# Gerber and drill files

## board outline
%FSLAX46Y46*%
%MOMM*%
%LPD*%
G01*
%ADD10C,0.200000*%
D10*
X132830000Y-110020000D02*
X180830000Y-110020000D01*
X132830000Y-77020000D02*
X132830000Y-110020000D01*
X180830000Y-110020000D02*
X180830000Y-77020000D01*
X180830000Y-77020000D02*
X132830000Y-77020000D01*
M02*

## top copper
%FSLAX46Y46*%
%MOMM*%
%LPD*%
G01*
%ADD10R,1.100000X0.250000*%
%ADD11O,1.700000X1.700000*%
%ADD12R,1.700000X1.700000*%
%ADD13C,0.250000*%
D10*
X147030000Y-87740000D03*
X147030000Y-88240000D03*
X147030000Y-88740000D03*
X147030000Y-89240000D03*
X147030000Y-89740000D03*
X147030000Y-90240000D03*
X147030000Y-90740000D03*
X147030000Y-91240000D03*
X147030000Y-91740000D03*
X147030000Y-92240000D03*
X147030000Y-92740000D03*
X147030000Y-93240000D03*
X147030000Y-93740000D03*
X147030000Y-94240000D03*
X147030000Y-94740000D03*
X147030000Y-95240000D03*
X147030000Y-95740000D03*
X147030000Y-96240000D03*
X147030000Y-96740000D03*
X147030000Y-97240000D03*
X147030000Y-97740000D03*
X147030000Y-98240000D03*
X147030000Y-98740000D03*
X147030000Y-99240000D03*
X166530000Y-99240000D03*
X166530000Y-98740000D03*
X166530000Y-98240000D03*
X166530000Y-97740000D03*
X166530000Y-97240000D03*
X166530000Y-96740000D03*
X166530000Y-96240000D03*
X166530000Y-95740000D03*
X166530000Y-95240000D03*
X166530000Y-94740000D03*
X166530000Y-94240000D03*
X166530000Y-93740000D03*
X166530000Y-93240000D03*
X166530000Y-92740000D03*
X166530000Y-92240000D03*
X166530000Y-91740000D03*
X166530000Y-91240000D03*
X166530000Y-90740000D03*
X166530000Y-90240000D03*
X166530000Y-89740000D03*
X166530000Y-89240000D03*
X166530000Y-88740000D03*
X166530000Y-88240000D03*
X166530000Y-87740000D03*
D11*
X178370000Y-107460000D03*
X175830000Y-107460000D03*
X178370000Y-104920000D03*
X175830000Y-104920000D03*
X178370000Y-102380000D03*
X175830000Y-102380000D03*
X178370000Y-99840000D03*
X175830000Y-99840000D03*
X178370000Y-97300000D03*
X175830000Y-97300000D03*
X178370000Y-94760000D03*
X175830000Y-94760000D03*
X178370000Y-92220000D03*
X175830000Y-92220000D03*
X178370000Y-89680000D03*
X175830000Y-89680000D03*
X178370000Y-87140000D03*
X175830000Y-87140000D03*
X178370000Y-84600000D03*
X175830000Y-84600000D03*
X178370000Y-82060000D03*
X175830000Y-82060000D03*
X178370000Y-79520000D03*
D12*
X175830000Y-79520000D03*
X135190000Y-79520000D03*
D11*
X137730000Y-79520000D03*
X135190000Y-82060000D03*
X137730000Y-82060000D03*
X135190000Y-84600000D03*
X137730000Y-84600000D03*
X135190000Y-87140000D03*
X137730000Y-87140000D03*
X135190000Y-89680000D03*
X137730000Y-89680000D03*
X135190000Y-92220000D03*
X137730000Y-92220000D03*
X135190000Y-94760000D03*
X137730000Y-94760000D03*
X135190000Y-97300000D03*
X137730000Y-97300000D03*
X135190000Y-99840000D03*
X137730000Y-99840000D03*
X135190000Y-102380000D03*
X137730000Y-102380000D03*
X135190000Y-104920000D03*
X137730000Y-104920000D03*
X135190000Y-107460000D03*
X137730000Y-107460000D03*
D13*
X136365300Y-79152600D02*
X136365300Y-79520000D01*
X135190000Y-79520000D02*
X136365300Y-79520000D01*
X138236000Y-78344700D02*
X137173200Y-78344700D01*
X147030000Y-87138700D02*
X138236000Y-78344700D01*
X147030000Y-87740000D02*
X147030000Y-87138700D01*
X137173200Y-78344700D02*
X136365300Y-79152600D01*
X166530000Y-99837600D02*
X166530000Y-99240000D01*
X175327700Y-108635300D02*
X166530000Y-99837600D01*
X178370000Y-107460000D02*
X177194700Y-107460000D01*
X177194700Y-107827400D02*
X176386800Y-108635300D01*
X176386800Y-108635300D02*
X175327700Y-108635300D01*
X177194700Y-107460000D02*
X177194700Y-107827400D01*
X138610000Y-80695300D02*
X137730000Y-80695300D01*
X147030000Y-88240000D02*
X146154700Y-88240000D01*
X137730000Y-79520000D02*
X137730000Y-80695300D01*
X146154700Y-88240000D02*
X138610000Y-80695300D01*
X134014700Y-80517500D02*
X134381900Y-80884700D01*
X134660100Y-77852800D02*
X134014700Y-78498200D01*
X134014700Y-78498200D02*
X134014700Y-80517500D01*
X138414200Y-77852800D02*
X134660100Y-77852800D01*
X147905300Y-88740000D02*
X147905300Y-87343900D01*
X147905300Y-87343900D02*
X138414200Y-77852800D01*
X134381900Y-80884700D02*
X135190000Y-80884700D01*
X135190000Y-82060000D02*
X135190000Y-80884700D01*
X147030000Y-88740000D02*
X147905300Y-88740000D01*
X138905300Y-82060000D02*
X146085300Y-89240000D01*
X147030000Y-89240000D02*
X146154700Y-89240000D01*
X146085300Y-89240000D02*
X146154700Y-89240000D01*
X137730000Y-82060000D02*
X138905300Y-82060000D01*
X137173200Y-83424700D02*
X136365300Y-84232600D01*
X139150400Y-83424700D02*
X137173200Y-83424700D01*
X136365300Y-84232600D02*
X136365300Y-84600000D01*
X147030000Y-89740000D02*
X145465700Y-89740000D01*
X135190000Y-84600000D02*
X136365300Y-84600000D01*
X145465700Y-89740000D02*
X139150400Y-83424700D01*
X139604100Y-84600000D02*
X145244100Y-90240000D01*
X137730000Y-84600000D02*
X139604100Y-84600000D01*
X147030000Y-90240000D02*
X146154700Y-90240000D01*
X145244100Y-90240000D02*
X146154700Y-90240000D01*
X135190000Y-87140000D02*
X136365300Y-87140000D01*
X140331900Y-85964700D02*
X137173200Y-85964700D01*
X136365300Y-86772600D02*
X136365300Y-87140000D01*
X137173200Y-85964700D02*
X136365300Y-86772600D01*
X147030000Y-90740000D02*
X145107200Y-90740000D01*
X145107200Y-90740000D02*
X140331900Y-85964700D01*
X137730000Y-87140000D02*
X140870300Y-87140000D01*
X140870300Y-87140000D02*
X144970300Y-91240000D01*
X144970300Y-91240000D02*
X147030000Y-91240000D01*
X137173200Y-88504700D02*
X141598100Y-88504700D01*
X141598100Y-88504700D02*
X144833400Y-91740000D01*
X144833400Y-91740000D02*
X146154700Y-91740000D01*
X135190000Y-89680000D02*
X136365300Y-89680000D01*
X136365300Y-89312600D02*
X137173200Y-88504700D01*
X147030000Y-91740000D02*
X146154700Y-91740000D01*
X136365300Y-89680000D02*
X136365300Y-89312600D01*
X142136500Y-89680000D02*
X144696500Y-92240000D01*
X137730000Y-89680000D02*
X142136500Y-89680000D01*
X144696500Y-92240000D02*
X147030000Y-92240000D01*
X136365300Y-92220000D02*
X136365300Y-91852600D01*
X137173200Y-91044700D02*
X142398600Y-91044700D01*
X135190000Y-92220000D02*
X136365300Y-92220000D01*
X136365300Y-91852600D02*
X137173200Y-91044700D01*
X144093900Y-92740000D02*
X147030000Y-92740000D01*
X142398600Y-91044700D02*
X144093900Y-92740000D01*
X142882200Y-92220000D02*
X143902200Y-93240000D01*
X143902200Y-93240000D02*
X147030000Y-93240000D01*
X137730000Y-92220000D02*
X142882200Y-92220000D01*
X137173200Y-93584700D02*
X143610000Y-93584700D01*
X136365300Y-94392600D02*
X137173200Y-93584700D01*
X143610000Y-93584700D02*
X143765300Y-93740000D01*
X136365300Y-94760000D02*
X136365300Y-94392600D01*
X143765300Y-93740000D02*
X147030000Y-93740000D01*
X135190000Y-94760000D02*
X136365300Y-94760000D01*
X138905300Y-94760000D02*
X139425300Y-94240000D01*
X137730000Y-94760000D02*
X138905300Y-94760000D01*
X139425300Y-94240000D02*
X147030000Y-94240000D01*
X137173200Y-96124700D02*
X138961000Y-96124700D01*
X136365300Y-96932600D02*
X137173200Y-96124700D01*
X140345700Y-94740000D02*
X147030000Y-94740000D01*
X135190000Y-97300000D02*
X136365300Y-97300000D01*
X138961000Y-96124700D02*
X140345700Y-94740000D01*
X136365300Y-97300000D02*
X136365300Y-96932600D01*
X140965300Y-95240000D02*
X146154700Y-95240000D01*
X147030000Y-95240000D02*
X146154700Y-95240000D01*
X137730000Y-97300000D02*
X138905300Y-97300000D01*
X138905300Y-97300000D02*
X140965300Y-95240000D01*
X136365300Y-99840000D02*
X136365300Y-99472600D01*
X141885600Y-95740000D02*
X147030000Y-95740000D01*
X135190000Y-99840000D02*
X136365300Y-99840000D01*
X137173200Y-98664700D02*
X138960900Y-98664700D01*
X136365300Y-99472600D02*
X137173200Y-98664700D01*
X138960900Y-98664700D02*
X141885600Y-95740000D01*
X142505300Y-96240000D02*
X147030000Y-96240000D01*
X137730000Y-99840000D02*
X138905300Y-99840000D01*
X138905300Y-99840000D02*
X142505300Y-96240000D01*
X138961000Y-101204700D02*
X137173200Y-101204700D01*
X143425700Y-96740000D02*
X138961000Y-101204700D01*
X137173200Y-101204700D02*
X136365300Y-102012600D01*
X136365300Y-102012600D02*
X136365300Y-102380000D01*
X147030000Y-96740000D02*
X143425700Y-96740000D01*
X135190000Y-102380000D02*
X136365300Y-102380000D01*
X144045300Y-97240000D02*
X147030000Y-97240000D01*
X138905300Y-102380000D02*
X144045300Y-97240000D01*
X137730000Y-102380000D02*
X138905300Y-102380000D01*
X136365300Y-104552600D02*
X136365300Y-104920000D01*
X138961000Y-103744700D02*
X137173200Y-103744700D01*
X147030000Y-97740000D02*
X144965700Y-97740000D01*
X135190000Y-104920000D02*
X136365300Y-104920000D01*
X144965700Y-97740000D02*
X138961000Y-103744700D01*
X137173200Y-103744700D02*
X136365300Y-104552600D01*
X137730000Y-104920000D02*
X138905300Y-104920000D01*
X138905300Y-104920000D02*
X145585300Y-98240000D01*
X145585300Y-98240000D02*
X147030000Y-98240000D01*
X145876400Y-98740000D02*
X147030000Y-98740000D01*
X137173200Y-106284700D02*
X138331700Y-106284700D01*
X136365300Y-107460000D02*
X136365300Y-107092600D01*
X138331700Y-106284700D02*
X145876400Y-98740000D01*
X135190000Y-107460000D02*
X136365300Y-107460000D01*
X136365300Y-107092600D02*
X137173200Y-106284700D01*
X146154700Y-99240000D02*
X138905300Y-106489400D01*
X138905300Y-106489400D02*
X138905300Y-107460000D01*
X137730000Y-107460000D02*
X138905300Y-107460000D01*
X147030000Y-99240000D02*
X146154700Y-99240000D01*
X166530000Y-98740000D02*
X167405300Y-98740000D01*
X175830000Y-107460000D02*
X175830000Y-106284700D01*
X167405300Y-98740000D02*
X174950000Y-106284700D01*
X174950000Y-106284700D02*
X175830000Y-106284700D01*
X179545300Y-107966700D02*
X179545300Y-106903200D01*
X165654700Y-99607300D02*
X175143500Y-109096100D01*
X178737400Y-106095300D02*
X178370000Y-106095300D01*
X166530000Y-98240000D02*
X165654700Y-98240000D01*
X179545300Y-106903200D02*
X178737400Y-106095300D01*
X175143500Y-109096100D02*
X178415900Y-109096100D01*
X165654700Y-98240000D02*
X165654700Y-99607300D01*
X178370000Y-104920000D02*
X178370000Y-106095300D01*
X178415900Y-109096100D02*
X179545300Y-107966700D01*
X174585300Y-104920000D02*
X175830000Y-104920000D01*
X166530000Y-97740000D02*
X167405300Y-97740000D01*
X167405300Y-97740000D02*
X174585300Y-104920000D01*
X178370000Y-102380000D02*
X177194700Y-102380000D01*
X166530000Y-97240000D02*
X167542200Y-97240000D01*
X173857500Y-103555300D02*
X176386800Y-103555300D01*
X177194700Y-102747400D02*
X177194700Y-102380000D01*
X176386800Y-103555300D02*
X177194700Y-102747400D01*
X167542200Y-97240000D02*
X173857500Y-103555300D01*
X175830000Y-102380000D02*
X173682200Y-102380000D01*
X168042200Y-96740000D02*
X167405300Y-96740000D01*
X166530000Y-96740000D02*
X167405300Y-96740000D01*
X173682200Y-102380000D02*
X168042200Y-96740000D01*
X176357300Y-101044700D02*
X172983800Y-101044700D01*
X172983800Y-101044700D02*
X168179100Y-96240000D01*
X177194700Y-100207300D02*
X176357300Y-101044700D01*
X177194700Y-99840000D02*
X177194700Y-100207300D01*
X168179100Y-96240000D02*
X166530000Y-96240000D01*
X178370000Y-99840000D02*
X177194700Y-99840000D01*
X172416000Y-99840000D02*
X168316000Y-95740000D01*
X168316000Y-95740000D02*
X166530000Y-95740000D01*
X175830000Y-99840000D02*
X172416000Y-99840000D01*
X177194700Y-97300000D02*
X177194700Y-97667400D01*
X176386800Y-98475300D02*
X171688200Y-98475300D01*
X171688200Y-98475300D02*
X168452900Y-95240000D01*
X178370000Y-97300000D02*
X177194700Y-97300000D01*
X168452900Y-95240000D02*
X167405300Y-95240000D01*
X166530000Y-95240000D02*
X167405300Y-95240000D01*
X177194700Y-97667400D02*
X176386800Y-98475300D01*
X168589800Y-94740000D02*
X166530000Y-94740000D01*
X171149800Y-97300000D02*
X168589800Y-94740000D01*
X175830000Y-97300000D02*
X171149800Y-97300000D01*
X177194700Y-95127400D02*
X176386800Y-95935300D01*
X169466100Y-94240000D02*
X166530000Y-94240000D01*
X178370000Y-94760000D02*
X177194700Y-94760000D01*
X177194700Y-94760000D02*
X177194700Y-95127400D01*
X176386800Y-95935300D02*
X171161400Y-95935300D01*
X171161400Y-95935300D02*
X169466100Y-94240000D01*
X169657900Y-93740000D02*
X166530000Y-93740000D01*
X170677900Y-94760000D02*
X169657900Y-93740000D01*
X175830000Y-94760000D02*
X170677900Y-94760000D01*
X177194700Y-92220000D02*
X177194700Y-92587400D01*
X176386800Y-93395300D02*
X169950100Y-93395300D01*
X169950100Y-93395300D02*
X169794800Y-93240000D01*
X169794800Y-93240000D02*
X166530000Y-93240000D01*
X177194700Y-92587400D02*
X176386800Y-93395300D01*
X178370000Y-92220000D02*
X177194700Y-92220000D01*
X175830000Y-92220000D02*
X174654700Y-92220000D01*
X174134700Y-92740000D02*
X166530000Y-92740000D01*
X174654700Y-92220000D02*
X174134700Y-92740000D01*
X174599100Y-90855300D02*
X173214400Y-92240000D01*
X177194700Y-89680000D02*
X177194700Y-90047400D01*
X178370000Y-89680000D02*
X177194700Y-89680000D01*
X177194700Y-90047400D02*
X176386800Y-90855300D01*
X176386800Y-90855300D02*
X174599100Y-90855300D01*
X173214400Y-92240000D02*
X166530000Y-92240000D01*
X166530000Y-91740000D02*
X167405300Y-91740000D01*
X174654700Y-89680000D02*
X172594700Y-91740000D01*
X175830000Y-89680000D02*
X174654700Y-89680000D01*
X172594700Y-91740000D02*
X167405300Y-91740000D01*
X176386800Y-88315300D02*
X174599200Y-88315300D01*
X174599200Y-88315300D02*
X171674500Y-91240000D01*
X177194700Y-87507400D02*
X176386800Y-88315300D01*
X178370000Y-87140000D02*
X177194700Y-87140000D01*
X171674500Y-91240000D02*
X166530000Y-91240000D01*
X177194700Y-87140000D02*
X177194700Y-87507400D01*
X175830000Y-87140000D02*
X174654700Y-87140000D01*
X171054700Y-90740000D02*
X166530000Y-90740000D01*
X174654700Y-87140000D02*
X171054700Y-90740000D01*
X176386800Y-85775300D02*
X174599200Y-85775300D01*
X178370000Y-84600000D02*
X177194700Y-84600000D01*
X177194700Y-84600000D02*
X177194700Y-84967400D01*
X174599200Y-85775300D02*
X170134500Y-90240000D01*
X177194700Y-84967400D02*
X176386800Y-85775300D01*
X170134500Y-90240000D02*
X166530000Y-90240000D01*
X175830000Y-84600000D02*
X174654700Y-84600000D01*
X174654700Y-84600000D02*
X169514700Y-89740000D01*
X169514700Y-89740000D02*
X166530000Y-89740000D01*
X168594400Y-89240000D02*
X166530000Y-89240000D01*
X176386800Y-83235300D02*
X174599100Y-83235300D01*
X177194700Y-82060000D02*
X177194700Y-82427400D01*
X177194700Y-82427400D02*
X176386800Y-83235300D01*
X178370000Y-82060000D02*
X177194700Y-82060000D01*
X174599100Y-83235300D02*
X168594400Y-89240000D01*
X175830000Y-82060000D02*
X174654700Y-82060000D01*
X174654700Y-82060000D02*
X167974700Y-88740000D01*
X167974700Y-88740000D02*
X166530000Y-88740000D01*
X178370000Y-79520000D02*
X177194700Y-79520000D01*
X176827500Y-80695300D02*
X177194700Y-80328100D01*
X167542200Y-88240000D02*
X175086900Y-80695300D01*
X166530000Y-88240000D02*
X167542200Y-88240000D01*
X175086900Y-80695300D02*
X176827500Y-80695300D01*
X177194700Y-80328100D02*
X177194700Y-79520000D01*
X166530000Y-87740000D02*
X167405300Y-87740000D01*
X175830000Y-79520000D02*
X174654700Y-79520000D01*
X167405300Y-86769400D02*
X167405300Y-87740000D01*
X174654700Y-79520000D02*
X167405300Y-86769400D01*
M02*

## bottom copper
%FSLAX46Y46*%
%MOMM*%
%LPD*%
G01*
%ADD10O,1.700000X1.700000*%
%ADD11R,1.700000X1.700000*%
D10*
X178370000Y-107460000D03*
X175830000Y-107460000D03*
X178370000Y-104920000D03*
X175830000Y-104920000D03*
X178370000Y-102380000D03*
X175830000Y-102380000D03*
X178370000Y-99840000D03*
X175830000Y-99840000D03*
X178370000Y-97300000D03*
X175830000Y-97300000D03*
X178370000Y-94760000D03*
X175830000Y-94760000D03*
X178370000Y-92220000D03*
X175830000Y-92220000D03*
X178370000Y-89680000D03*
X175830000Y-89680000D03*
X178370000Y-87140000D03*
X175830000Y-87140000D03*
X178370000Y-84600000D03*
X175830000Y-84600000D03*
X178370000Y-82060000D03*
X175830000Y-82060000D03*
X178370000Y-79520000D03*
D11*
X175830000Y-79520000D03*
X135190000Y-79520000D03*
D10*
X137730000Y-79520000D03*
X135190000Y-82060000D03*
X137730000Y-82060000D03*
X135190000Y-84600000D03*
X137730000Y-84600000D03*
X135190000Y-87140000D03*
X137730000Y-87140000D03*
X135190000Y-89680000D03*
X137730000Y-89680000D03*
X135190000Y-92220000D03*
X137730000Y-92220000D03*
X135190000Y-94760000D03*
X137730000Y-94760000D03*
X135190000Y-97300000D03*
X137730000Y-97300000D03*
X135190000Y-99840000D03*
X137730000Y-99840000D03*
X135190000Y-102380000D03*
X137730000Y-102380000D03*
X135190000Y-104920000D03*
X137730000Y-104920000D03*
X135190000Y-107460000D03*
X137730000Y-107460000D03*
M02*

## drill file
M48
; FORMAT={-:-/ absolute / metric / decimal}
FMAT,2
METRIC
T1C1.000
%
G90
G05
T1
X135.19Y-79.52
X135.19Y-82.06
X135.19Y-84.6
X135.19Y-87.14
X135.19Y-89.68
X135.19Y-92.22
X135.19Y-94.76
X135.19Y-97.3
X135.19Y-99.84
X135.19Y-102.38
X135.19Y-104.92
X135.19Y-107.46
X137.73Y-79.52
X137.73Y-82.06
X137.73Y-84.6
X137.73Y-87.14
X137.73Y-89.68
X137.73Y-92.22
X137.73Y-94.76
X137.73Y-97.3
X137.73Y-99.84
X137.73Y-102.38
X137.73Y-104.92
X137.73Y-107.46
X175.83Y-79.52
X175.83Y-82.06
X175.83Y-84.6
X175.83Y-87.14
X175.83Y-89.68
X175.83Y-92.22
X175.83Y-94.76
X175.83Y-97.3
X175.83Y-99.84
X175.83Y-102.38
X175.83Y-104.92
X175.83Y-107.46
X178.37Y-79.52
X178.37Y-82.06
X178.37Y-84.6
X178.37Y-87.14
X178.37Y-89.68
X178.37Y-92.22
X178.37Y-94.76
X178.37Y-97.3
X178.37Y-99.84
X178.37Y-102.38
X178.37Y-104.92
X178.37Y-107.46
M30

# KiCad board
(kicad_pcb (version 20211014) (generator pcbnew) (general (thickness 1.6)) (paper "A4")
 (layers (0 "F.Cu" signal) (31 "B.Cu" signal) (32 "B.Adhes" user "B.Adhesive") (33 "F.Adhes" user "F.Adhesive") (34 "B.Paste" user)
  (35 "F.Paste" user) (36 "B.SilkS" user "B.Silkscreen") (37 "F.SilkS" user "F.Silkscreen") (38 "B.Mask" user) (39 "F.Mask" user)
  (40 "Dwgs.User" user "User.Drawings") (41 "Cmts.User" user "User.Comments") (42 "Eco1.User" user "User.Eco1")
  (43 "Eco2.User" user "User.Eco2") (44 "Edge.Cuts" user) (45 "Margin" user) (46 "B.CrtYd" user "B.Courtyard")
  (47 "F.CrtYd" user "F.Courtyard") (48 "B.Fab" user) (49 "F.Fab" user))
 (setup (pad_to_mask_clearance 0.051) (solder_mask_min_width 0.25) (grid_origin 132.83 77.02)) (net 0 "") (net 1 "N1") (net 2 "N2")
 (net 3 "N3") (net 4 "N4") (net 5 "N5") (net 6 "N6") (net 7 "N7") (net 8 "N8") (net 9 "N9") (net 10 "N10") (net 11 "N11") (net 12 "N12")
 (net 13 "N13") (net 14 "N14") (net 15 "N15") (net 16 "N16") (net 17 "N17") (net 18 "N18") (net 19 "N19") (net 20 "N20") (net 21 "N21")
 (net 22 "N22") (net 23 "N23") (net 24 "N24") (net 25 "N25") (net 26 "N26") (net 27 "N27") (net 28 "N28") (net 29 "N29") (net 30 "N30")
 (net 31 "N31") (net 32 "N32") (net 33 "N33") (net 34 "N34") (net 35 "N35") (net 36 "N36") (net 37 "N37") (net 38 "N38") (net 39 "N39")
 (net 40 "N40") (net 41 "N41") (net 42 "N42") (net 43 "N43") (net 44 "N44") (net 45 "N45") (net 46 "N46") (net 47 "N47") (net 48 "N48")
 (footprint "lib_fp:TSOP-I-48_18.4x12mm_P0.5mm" (layer "F.Cu") (at 156.78 93.49)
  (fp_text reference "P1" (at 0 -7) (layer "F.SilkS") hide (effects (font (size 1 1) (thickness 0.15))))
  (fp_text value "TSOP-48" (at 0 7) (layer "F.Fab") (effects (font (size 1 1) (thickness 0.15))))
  (pad "1" smd rect locked (at -9.75 -5.75) (size 1.1 0.25) (layers "F.Cu" "F.Paste" "F.Mask") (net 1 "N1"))
  (pad "2" smd rect locked (at -9.75 -5.25) (size 1.1 0.25) (layers "F.Cu" "F.Paste" "F.Mask") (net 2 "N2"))
  (pad "3" smd rect locked (at -9.75 -4.75) (size 1.1 0.25) (layers "F.Cu" "F.Paste" "F.Mask") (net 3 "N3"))
  (pad "4" smd rect locked (at -9.75 -4.25) (size 1.1 0.25) (layers "F.Cu" "F.Paste" "F.Mask") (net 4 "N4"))
  (pad "5" smd rect locked (at -9.75 -3.75) (size 1.1 0.25) (layers "F.Cu" "F.Paste" "F.Mask") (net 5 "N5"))
  (pad "6" smd rect locked (at -9.75 -3.25) (size 1.1 0.25) (layers "F.Cu" "F.Paste" "F.Mask") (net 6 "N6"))
  (pad "7" smd rect locked (at -9.75 -2.75) (size 1.1 0.25) (layers "F.Cu" "F.Paste" "F.Mask") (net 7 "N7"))
  (pad "8" smd rect locked (at -9.75 -2.25) (size 1.1 0.25) (layers "F.Cu" "F.Paste" "F.Mask") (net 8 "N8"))
  (pad "9" smd rect locked (at -9.75 -1.75) (size 1.1 0.25) (layers "F.Cu" "F.Paste" "F.Mask") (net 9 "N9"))
  (pad "10" smd rect locked (at -9.75 -1.25) (size 1.1 0.25) (layers "F.Cu" "F.Paste" "F.Mask") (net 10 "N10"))
  (pad "11" smd rect locked (at -9.75 -0.75) (size 1.1 0.25) (layers "F.Cu" "F.Paste" "F.Mask") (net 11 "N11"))
  (pad "12" smd rect locked (at -9.75 -0.25) (size 1.1 0.25) (layers "F.Cu" "F.Paste" "F.Mask") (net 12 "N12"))
  (pad "13" smd rect locked (at -9.75 0.25) (size 1.1 0.25) (layers "F.Cu" "F.Paste" "F.Mask") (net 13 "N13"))
  (pad "14" smd rect locked (at -9.75 0.75) (size 1.1 0.25) (layers "F.Cu" "F.Paste" "F.Mask") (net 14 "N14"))
  (pad "15" smd rect locked (at -9.75 1.25) (size 1.1 0.25) (layers "F.Cu" "F.Paste" "F.Mask") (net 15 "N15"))
  (pad "16" smd rect locked (at -9.75 1.75) (size 1.1 0.25) (layers "F.Cu" "F.Paste" "F.Mask") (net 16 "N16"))
  (pad "17" smd rect locked (at -9.75 2.25) (size 1.1 0.25) (layers "F.Cu" "F.Paste" "F.Mask") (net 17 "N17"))
  (pad "18" smd rect locked (at -9.75 2.75) (size 1.1 0.25) (layers "F.Cu" "F.Paste" "F.Mask") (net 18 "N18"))
  (pad "19" smd rect locked (at -9.75 3.25) (size 1.1 0.25) (layers "F.Cu" "F.Paste" "F.Mask") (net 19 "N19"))
  (pad "20" smd rect locked (at -9.75 3.75) (size 1.1 0.25) (layers "F.Cu" "F.Paste" "F.Mask") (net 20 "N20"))
  (pad "21" smd rect locked (at -9.75 4.25) (size 1.1 0.25) (layers "F.Cu" "F.Paste" "F.Mask") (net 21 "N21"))
  (pad "22" smd rect locked (at -9.75 4.75) (size 1.1 0.25) (layers "F.Cu" "F.Paste" "F.Mask") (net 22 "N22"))
  (pad "23" smd rect locked (at -9.75 5.25) (size 1.1 0.25) (layers "F.Cu" "F.Paste" "F.Mask") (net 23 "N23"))
  (pad "24" smd rect locked (at -9.75 5.75) (size 1.1 0.25) (layers "F.Cu" "F.Paste" "F.Mask") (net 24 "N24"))
  (pad "25" smd rect locked (at 9.75 5.75) (size 1.1 0.25) (layers "F.Cu" "F.Paste" "F.Mask") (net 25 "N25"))
  (pad "26" smd rect locked (at 9.75 5.25) (size 1.1 0.25) (layers "F.Cu" "F.Paste" "F.Mask") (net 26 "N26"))
  (pad "27" smd rect locked (at 9.75 4.75) (size 1.1 0.25) (layers "F.Cu" "F.Paste" "F.Mask") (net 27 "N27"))
  (pad "28" smd rect locked (at 9.75 4.25) (size 1.1 0.25) (layers "F.Cu" "F.Paste" "F.Mask") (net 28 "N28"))
  (pad "29" smd rect locked (at 9.75 3.75) (size 1.1 0.25) (layers "F.Cu" "F.Paste" "F.Mask") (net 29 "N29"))
  (pad "30" smd rect locked (at 9.75 3.25) (size 1.1 0.25) (layers "F.Cu" "F.Paste" "F.Mask") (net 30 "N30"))
  (pad "31" smd rect locked (at 9.75 2.75) (size 1.1 0.25) (layers "F.Cu" "F.Paste" "F.Mask") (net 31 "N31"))
  (pad "32" smd rect locked (at 9.75 2.25) (size 1.1 0.25) (layers "F.Cu" "F.Paste" "F.Mask") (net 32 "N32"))
  (pad "33" smd rect locked (at 9.75 1.75) (size 1.1 0.25) (layers "F.Cu" "F.Paste" "F.Mask") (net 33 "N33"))
  (pad "34" smd rect locked (at 9.75 1.25) (size 1.1 0.25) (layers "F.Cu" "F.Paste" "F.Mask") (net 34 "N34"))
  (pad "35" smd rect locked (at 9.75 0.75) (size 1.1 0.25) (layers "F.Cu" "F.Paste" "F.Mask") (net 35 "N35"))
  (pad "36" smd rect locked (at 9.75 0.25) (size 1.1 0.25) (layers "F.Cu" "F.Paste" "F.Mask") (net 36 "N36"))
  (pad "37" smd rect locked (at 9.75 -0.25) (size 1.1 0.25) (layers "F.Cu" "F.Paste" "F.Mask") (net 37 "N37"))
  (pad "38" smd rect locked (at 9.75 -0.75) (size 1.1 0.25) (layers "F.Cu" "F.Paste" "F.Mask") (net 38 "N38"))
  (pad "39" smd rect locked (at 9.75 -1.25) (size 1.1 0.25) (layers "F.Cu" "F.Paste" "F.Mask") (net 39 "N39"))
  (pad "40" smd rect locked (at 9.75 -1.75) (size 1.1 0.25) (layers "F.Cu" "F.Paste" "F.Mask") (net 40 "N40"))
  (pad "41" smd rect locked (at 9.75 -2.25) (size 1.1 0.25) (layers "F.Cu" "F.Paste" "F.Mask") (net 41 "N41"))
  (pad "42" smd rect locked (at 9.75 -2.75) (size 1.1 0.25) (layers "F.Cu" "F.Paste" "F.Mask") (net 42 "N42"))
  (pad "43" smd rect locked (at 9.75 -3.25) (size 1.1 0.25) (layers "F.Cu" "F.Paste" "F.Mask") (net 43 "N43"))
  (pad "44" smd rect locked (at 9.75 -3.75) (size 1.1 0.25) (layers "F.Cu" "F.Paste" "F.Mask") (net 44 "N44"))
  (pad "45" smd rect locked (at 9.75 -4.25) (size 1.1 0.25) (layers "F.Cu" "F.Paste" "F.Mask") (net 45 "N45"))
  (pad "46" smd rect locked (at 9.75 -4.75) (size 1.1 0.25) (layers "F.Cu" "F.Paste" "F.Mask") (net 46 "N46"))
  (pad "47" smd rect locked (at 9.75 -5.25) (size 1.1 0.25) (layers "F.Cu" "F.Paste" "F.Mask") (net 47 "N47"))
  (pad "48" smd rect locked (at 9.75 -5.75) (size 1.1 0.25) (layers "F.Cu" "F.Paste" "F.Mask") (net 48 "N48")))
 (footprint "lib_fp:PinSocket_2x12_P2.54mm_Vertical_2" (layer "B.Cu") (at 175.83 79.52 180)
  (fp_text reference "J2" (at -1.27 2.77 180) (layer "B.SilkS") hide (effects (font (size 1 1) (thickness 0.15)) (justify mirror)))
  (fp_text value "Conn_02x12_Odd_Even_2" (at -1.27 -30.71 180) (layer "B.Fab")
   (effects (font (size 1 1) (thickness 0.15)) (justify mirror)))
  (pad "25" thru_hole oval locked (at -2.54 -27.94 180) (size 1.7 1.7) (drill 1) (layers *.Cu *.Mask) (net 25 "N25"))
  (pad "26" thru_hole oval locked (at 0 -27.94 180) (size 1.7 1.7) (drill 1) (layers *.Cu *.Mask) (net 26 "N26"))
  (pad "27" thru_hole oval locked (at -2.54 -25.4 180) (size 1.7 1.7) (drill 1) (layers *.Cu *.Mask) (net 27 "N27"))
  (pad "28" thru_hole oval locked (at 0 -25.4 180) (size 1.7 1.7) (drill 1) (layers *.Cu *.Mask) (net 28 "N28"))
  (pad "29" thru_hole oval locked (at -2.54 -22.86 180) (size 1.7 1.7) (drill 1) (layers *.Cu *.Mask) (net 29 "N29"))
  (pad "30" thru_hole oval locked (at 0 -22.86 180) (size 1.7 1.7) (drill 1) (layers *.Cu *.Mask) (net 30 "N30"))
  (pad "31" thru_hole oval locked (at -2.54 -20.32 180) (size 1.7 1.7) (drill 1) (layers *.Cu *.Mask) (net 31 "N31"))
  (pad "32" thru_hole oval locked (at 0 -20.32 180) (size 1.7 1.7) (drill 1) (layers *.Cu *.Mask) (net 32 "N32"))
  (pad "33" thru_hole oval locked (at -2.54 -17.78 180) (size 1.7 1.7) (drill 1) (layers *.Cu *.Mask) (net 33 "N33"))
  (pad "34" thru_hole oval locked (at 0 -17.78 180) (size 1.7 1.7) (drill 1) (layers *.Cu *.Mask) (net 34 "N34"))
  (pad "35" thru_hole oval locked (at -2.54 -15.24 180) (size 1.7 1.7) (drill 1) (layers *.Cu *.Mask) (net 35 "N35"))
  (pad "36" thru_hole oval locked (at 0 -15.24 180) (size 1.7 1.7) (drill 1) (layers *.Cu *.Mask) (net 36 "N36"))
  (pad "37" thru_hole oval locked (at -2.54 -12.7 180) (size 1.7 1.7) (drill 1) (layers *.Cu *.Mask) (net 37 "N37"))
  (pad "38" thru_hole oval locked (at 0 -12.7 180) (size 1.7 1.7) (drill 1) (layers *.Cu *.Mask) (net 38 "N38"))
  (pad "39" thru_hole oval locked (at -2.54 -10.16 180) (size 1.7 1.7) (drill 1) (layers *.Cu *.Mask) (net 39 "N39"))
  (pad "40" thru_hole oval locked (at 0 -10.16 180) (size 1.7 1.7) (drill 1) (layers *.Cu *.Mask) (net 40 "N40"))
  (pad "41" thru_hole oval locked (at -2.54 -7.62 180) (size 1.7 1.7) (drill 1) (layers *.Cu *.Mask) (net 41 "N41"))
  (pad "42" thru_hole oval locked (at 0 -7.62 180) (size 1.7 1.7) (drill 1) (layers *.Cu *.Mask) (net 42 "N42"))
  (pad "43" thru_hole oval locked (at -2.54 -5.08 180) (size 1.7 1.7) (drill 1) (layers *.Cu *.Mask) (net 43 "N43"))
  (pad "44" thru_hole oval locked (at 0 -5.08 180) (size 1.7 1.7) (drill 1) (layers *.Cu *.Mask) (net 44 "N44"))
  (pad "45" thru_hole oval locked (at -2.54 -2.54 180) (size 1.7 1.7) (drill 1) (layers *.Cu *.Mask) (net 45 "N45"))
  (pad "46" thru_hole oval locked (at 0 -2.54 180) (size 1.7 1.7) (drill 1) (layers *.Cu *.Mask) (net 46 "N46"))
  (pad "47" thru_hole oval locked (at -2.54 0 180) (size 1.7 1.7) (drill 1) (layers *.Cu *.Mask) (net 47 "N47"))
  (pad "48" thru_hole rect locked (at 0 0 180) (size 1.7 1.7) (drill 1) (layers *.Cu *.Mask) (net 48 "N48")))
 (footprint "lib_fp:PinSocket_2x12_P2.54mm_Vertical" (layer "B.Cu") (at 135.19 79.52 180)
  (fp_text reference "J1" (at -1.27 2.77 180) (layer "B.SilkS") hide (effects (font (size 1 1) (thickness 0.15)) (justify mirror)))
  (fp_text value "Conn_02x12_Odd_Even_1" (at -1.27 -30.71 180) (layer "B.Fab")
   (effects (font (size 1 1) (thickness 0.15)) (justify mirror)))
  (pad "1" thru_hole rect locked (at 0 0 180) (size 1.7 1.7) (drill 1) (layers *.Cu *.Mask) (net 1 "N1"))
  (pad "2" thru_hole oval locked (at -2.54 0 180) (size 1.7 1.7) (drill 1) (layers *.Cu *.Mask) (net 2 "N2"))
  (pad "3" thru_hole oval locked (at 0 -2.54 180) (size 1.7 1.7) (drill 1) (layers *.Cu *.Mask) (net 3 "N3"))
  (pad "4" thru_hole oval locked (at -2.54 -2.54 180) (size 1.7 1.7) (drill 1) (layers *.Cu *.Mask) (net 4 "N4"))
  (pad "5" thru_hole oval locked (at 0 -5.08 180) (size 1.7 1.7) (drill 1) (layers *.Cu *.Mask) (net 5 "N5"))
  (pad "6" thru_hole oval locked (at -2.54 -5.08 180) (size 1.7 1.7) (drill 1) (layers *.Cu *.Mask) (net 6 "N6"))
  (pad "7" thru_hole oval locked (at 0 -7.62 180) (size 1.7 1.7) (drill 1) (layers *.Cu *.Mask) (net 7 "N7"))
  (pad "8" thru_hole oval locked (at -2.54 -7.62 180) (size 1.7 1.7) (drill 1) (layers *.Cu *.Mask) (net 8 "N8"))
  (pad "9" thru_hole oval locked (at 0 -10.16 180) (size 1.7 1.7) (drill 1) (layers *.Cu *.Mask) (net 9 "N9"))
  (pad "10" thru_hole oval locked (at -2.54 -10.16 180) (size 1.7 1.7) (drill 1) (layers *.Cu *.Mask) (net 10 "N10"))
  (pad "11" thru_hole oval locked (at 0 -12.7 180) (size 1.7 1.7) (drill 1) (layers *.Cu *.Mask) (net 11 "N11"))
  (pad "12" thru_hole oval locked (at -2.54 -12.7 180) (size 1.7 1.7) (drill 1) (layers *.Cu *.Mask) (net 12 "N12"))
  (pad "13" thru_hole oval locked (at 0 -15.24 180) (size 1.7 1.7) (drill 1) (layers *.Cu *.Mask) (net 13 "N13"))
  (pad "14" thru_hole oval locked (at -2.54 -15.24 180) (size 1.7 1.7) (drill 1) (layers *.Cu *.Mask) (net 14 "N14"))
  (pad "15" thru_hole oval locked (at 0 -17.78 180) (size 1.7 1.7) (drill 1) (layers *.Cu *.Mask) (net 15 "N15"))
  (pad "16" thru_hole oval locked (at -2.54 -17.78 180) (size 1.7 1.7) (drill 1) (layers *.Cu *.Mask) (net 16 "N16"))
  (pad "17" thru_hole oval locked (at 0 -20.32 180) (size 1.7 1.7) (drill 1) (layers *.Cu *.Mask) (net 17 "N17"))
  (pad "18" thru_hole oval locked (at -2.54 -20.32 180) (size 1.7 1.7) (drill 1) (layers *.Cu *.Mask) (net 18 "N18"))
  (pad "19" thru_hole oval locked (at 0 -22.86 180) (size 1.7 1.7) (drill 1) (layers *.Cu *.Mask) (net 19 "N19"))
  (pad "20" thru_hole oval locked (at -2.54 -22.86 180) (size 1.7 1.7) (drill 1) (layers *.Cu *.Mask) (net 20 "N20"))
  (pad "21" thru_hole oval locked (at 0 -25.4 180) (size 1.7 1.7) (drill 1) (layers *.Cu *.Mask) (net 21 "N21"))
  (pad "22" thru_hole oval locked (at -2.54 -25.4 180) (size 1.7 1.7) (drill 1) (layers *.Cu *.Mask) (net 22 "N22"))
  (pad "23" thru_hole oval locked (at 0 -27.94 180) (size 1.7 1.7) (drill 1) (layers *.Cu *.Mask) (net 23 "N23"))
  (pad "24" thru_hole oval locked (at -2.54 -27.94 180) (size 1.7 1.7) (drill 1) (layers *.Cu *.Mask) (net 24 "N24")))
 (gr_line (start 132.83 110.02) (end 180.83 110.02) (layer "Edge.Cuts") (width 0.2))
 (gr_line (start 132.83 77.02) (end 132.83 110.02) (layer "Edge.Cuts") (width 0.2))
 (gr_line (start 180.83 110.02) (end 180.83 77.02) (layer "Edge.Cuts") (width 0.2))
 (gr_line (start 180.83 77.02) (end 132.83 77.02) (layer "Edge.Cuts") (width 0.2))
 (segment (start 136.3653 79.1526) (end 136.3653 79.52) (width 0.25) (layer "F.Cu") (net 1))
 (segment (start 135.19 79.52) (end 136.3653 79.52) (width 0.25) (layer "F.Cu") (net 1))
 (segment (start 138.236 78.3447) (end 137.1732 78.3447) (width 0.25) (layer "F.Cu") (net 1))
 (segment (start 147.03 87.1387) (end 138.236 78.3447) (width 0.25) (layer "F.Cu") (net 1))
 (segment (start 147.03 87.74) (end 147.03 87.1387) (width 0.25) (layer "F.Cu") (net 1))
 (segment (start 137.1732 78.3447) (end 136.3653 79.1526) (width 0.25) (layer "F.Cu") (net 1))
 (segment (start 166.53 99.8376) (end 166.53 99.24) (width 0.25) (layer "F.Cu") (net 25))
 (segment (start 175.3277 108.6353) (end 166.53 99.8376) (width 0.25) (layer "F.Cu") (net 25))
 (segment (start 178.37 107.46) (end 177.1947 107.46) (width 0.25) (layer "F.Cu") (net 25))
 (segment (start 177.1947 107.8274) (end 176.3868 108.6353) (width 0.25) (layer "F.Cu") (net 25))
 (segment (start 176.3868 108.6353) (end 175.3277 108.6353) (width 0.25) (layer "F.Cu") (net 25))
 (segment (start 177.1947 107.46) (end 177.1947 107.8274) (width 0.25) (layer "F.Cu") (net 25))
 (segment (start 138.61 80.6953) (end 137.73 80.6953) (width 0.25) (layer "F.Cu") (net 2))
 (segment (start 147.03 88.24) (end 146.1547 88.24) (width 0.25) (layer "F.Cu") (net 2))
 (segment (start 137.73 79.52) (end 137.73 80.6953) (width 0.25) (layer "F.Cu") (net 2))
 (segment (start 146.1547 88.24) (end 138.61 80.6953) (width 0.25) (layer "F.Cu") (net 2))
 (segment (start 134.0147 80.5175) (end 134.3819 80.8847) (width 0.25) (layer "F.Cu") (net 3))
 (segment (start 134.6601 77.8528) (end 134.0147 78.4982) (width 0.25) (layer "F.Cu") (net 3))
 (segment (start 134.0147 78.4982) (end 134.0147 80.5175) (width 0.25) (layer "F.Cu") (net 3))
 (segment (start 138.4142 77.8528) (end 134.6601 77.8528) (width 0.25) (layer "F.Cu") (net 3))
 (segment (start 147.9053 88.74) (end 147.9053 87.3439) (width 0.25) (layer "F.Cu") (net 3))
 (segment (start 147.9053 87.3439) (end 138.4142 77.8528) (width 0.25) (layer "F.Cu") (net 3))
 (segment (start 134.3819 80.8847) (end 135.19 80.8847) (width 0.25) (layer "F.Cu") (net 3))
 (segment (start 135.19 82.06) (end 135.19 80.8847) (width 0.25) (layer "F.Cu") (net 3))
 (segment (start 147.03 88.74) (end 147.9053 88.74) (width 0.25) (layer "F.Cu") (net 3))
 (segment (start 138.9053 82.06) (end 146.0853 89.24) (width 0.25) (layer "F.Cu") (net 4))
 (segment (start 147.03 89.24) (end 146.1547 89.24) (width 0.25) (layer "F.Cu") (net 4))
 (segment (start 146.0853 89.24) (end 146.1547 89.24) (width 0.25) (layer "F.Cu") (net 4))
 (segment (start 137.73 82.06) (end 138.9053 82.06) (width 0.25) (layer "F.Cu") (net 4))
 (segment (start 137.1732 83.4247) (end 136.3653 84.2326) (width 0.25) (layer "F.Cu") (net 5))
 (segment (start 139.1504 83.4247) (end 137.1732 83.4247) (width 0.25) (layer "F.Cu") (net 5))
 (segment (start 136.3653 84.2326) (end 136.3653 84.6) (width 0.25) (layer "F.Cu") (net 5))
 (segment (start 147.03 89.74) (end 145.4657 89.74) (width 0.25) (layer "F.Cu") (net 5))
 (segment (start 135.19 84.6) (end 136.3653 84.6) (width 0.25) (layer "F.Cu") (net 5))
 (segment (start 145.4657 89.74) (end 139.1504 83.4247) (width 0.25) (layer "F.Cu") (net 5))
 (segment (start 139.6041 84.6) (end 145.2441 90.24) (width 0.25) (layer "F.Cu") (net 6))
 (segment (start 137.73 84.6) (end 139.6041 84.6) (width 0.25) (layer "F.Cu") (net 6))
 (segment (start 147.03 90.24) (end 146.1547 90.24) (width 0.25) (layer "F.Cu") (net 6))
 (segment (start 145.2441 90.24) (end 146.1547 90.24) (width 0.25) (layer "F.Cu") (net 6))
 (segment (start 135.19 87.14) (end 136.3653 87.14) (width 0.25) (layer "F.Cu") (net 7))
 (segment (start 140.3319 85.9647) (end 137.1732 85.9647) (width 0.25) (layer "F.Cu") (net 7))
 (segment (start 136.3653 86.7726) (end 136.3653 87.14) (width 0.25) (layer "F.Cu") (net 7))
 (segment (start 137.1732 85.9647) (end 136.3653 86.7726) (width 0.25) (layer "F.Cu") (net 7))
 (segment (start 147.03 90.74) (end 145.1072 90.74) (width 0.25) (layer "F.Cu") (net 7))
 (segment (start 145.1072 90.74) (end 140.3319 85.9647) (width 0.25) (layer "F.Cu") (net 7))
 (segment (start 137.73 87.14) (end 140.8703 87.14) (width 0.25) (layer "F.Cu") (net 8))
 (segment (start 140.8703 87.14) (end 144.9703 91.24) (width 0.25) (layer "F.Cu") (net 8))
 (segment (start 144.9703 91.24) (end 147.03 91.24) (width 0.25) (layer "F.Cu") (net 8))
 (segment (start 137.1732 88.5047) (end 141.5981 88.5047) (width 0.25) (layer "F.Cu") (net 9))
 (segment (start 141.5981 88.5047) (end 144.8334 91.74) (width 0.25) (layer "F.Cu") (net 9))
 (segment (start 144.8334 91.74) (end 146.1547 91.74) (width 0.25) (layer "F.Cu") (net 9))
 (segment (start 135.19 89.68) (end 136.3653 89.68) (width 0.25) (layer "F.Cu") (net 9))
 (segment (start 136.3653 89.3126) (end 137.1732 88.5047) (width 0.25) (layer "F.Cu") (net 9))
 (segment (start 147.03 91.74) (end 146.1547 91.74) (width 0.25) (layer "F.Cu") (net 9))
 (segment (start 136.3653 89.68) (end 136.3653 89.3126) (width 0.25) (layer "F.Cu") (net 9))
 (segment (start 142.1365 89.68) (end 144.6965 92.24) (width 0.25) (layer "F.Cu") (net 10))
 (segment (start 137.73 89.68) (end 142.1365 89.68) (width 0.25) (layer "F.Cu") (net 10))
 (segment (start 144.6965 92.24) (end 147.03 92.24) (width 0.25) (layer "F.Cu") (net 10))
 (segment (start 136.3653 92.22) (end 136.3653 91.8526) (width 0.25) (layer "F.Cu") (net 11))
 (segment (start 137.1732 91.0447) (end 142.3986 91.0447) (width 0.25) (layer "F.Cu") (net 11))
 (segment (start 135.19 92.22) (end 136.3653 92.22) (width 0.25) (layer "F.Cu") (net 11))
 (segment (start 136.3653 91.8526) (end 137.1732 91.0447) (width 0.25) (layer "F.Cu") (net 11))
 (segment (start 144.0939 92.74) (end 147.03 92.74) (width 0.25) (layer "F.Cu") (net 11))
 (segment (start 142.3986 91.0447) (end 144.0939 92.74) (width 0.25) (layer "F.Cu") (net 11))
 (segment (start 142.8822 92.22) (end 143.9022 93.24) (width 0.25) (layer "F.Cu") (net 12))
 (segment (start 143.9022 93.24) (end 147.03 93.24) (width 0.25) (layer "F.Cu") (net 12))
 (segment (start 137.73 92.22) (end 142.8822 92.22) (width 0.25) (layer "F.Cu") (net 12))
 (segment (start 137.1732 93.5847) (end 143.61 93.5847) (width 0.25) (layer "F.Cu") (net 13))
 (segment (start 136.3653 94.3926) (end 137.1732 93.5847) (width 0.25) (layer "F.Cu") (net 13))
 (segment (start 143.61 93.5847) (end 143.7653 93.74) (width 0.25) (layer "F.Cu") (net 13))
 (segment (start 136.3653 94.76) (end 136.3653 94.3926) (width 0.25) (layer "F.Cu") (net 13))
 (segment (start 143.7653 93.74) (end 147.03 93.74) (width 0.25) (layer "F.Cu") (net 13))
 (segment (start 135.19 94.76) (end 136.3653 94.76) (width 0.25) (layer "F.Cu") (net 13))
 (segment (start 138.9053 94.76) (end 139.4253 94.24) (width 0.25) (layer "F.Cu") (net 14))
 (segment (start 137.73 94.76) (end 138.9053 94.76) (width 0.25) (layer "F.Cu") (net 14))
 (segment (start 139.4253 94.24) (end 147.03 94.24) (width 0.25) (layer "F.Cu") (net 14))
 (segment (start 137.1732 96.1247) (end 138.961 96.1247) (width 0.25) (layer "F.Cu") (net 15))
 (segment (start 136.3653 96.9326) (end 137.1732 96.1247) (width 0.25) (layer "F.Cu") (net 15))
 (segment (start 140.3457 94.74) (end 147.03 94.74) (width 0.25) (layer "F.Cu") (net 15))
 (segment (start 135.19 97.3) (end 136.3653 97.3) (width 0.25) (layer "F.Cu") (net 15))
 (segment (start 138.961 96.1247) (end 140.3457 94.74) (width 0.25) (layer "F.Cu") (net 15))
 (segment (start 136.3653 97.3) (end 136.3653 96.9326) (width 0.25) (layer "F.Cu") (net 15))
 (segment (start 140.9653 95.24) (end 146.1547 95.24) (width 0.25) (layer "F.Cu") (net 16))
 (segment (start 147.03 95.24) (end 146.1547 95.24) (width 0.25) (layer "F.Cu") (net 16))
 (segment (start 137.73 97.3) (end 138.9053 97.3) (width 0.25) (layer "F.Cu") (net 16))
 (segment (start 138.9053 97.3) (end 140.9653 95.24) (width 0.25) (layer "F.Cu") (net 16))
 (segment (start 136.3653 99.84) (end 136.3653 99.4726) (width 0.25) (layer "F.Cu") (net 17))
 (segment (start 141.8856 95.74) (end 147.03 95.74) (width 0.25) (layer "F.Cu") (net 17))
 (segment (start 135.19 99.84) (end 136.3653 99.84) (width 0.25) (layer "F.Cu") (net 17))
 (segment (start 137.1732 98.6647) (end 138.9609 98.6647) (width 0.25) (layer "F.Cu") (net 17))
 (segment (start 136.3653 99.4726) (end 137.1732 98.6647) (width 0.25) (layer "F.Cu") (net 17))
 (segment (start 138.9609 98.6647) (end 141.8856 95.74) (width 0.25) (layer "F.Cu") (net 17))
 (segment (start 142.5053 96.24) (end 147.03 96.24) (width 0.25) (layer "F.Cu") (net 18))
 (segment (start 137.73 99.84) (end 138.9053 99.84) (width 0.25) (layer "F.Cu") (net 18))
 (segment (start 138.9053 99.84) (end 142.5053 96.24) (width 0.25) (layer "F.Cu") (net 18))
 (segment (start 138.961 101.2047) (end 137.1732 101.2047) (width 0.25) (layer "F.Cu") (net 19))
 (segment (start 143.4257 96.74) (end 138.961 101.2047) (width 0.25) (layer "F.Cu") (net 19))
 (segment (start 137.1732 101.2047) (end 136.3653 102.0126) (width 0.25) (layer "F.Cu") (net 19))
 (segment (start 136.3653 102.0126) (end 136.3653 102.38) (width 0.25) (layer "F.Cu") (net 19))
 (segment (start 147.03 96.74) (end 143.4257 96.74) (width 0.25) (layer "F.Cu") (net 19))
 (segment (start 135.19 102.38) (end 136.3653 102.38) (width 0.25) (layer "F.Cu") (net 19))
 (segment (start 144.0453 97.24) (end 147.03 97.24) (width 0.25) (layer "F.Cu") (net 20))
 (segment (start 138.9053 102.38) (end 144.0453 97.24) (width 0.25) (layer "F.Cu") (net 20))
 (segment (start 137.73 102.38) (end 138.9053 102.38) (width 0.25) (layer "F.Cu") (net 20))
 (segment (start 136.3653 104.5526) (end 136.3653 104.92) (width 0.25) (layer "F.Cu") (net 21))
 (segment (start 138.961 103.7447) (end 137.1732 103.7447) (width 0.25) (layer "F.Cu") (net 21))
 (segment (start 147.03 97.74) (end 144.9657 97.74) (width 0.25) (layer "F.Cu") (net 21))
 (segment (start 135.19 104.92) (end 136.3653 104.92) (width 0.25) (layer "F.Cu") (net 21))
 (segment (start 144.9657 97.74) (end 138.961 103.7447) (width 0.25) (layer "F.Cu") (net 21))
 (segment (start 137.1732 103.7447) (end 136.3653 104.5526) (width 0.25) (layer "F.Cu") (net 21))
 (segment (start 137.73 104.92) (end 138.9053 104.92) (width 0.25) (layer "F.Cu") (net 22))
 (segment (start 138.9053 104.92) (end 145.5853 98.24) (width 0.25) (layer "F.Cu") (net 22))
 (segment (start 145.5853 98.24) (end 147.03 98.24) (width 0.25) (layer "F.Cu") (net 22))
 (segment (start 145.8764 98.74) (end 147.03 98.74) (width 0.25) (layer "F.Cu") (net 23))
 (segment (start 137.1732 106.2847) (end 138.3317 106.2847) (width 0.25) (layer "F.Cu") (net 23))
 (segment (start 136.3653 107.46) (end 136.3653 107.0926) (width 0.25) (layer "F.Cu") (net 23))
 (segment (start 138.3317 106.2847) (end 145.8764 98.74) (width 0.25) (layer "F.Cu") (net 23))
 (segment (start 135.19 107.46) (end 136.3653 107.46) (width 0.25) (layer "F.Cu") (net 23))
 (segment (start 136.3653 107.0926) (end 137.1732 106.2847) (width 0.25) (layer "F.Cu") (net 23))
 (segment (start 146.1547 99.24) (end 138.9053 106.4894) (width 0.25) (layer "F.Cu") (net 24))
 (segment (start 138.9053 106.4894) (end 138.9053 107.46) (width 0.25) (layer "F.Cu") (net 24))
 (segment (start 137.73 107.46) (end 138.9053 107.46) (width 0.25) (layer "F.Cu") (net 24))
 (segment (start 147.03 99.24) (end 146.1547 99.24) (width 0.25) (layer "F.Cu") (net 24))
 (segment (start 166.53 98.74) (end 167.4053 98.74) (width 0.25) (layer "F.Cu") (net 26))
 (segment (start 175.83 107.46) (end 175.83 106.2847) (width 0.25) (layer "F.Cu") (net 26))
 (segment (start 167.4053 98.74) (end 174.95 106.2847) (width 0.25) (layer "F.Cu") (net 26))
 (segment (start 174.95 106.2847) (end 175.83 106.2847) (width 0.25) (layer "F.Cu") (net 26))
 (segment (start 179.5453 107.9667) (end 179.5453 106.9032) (width 0.25) (layer "F.Cu") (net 27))
 (segment (start 165.6547 99.6073) (end 175.1435 109.0961) (width 0.25) (layer "F.Cu") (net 27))
 (segment (start 178.7374 106.0953) (end 178.37 106.0953) (width 0.25) (layer "F.Cu") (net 27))
 (segment (start 166.53 98.24) (end 165.6547 98.24) (width 0.25) (layer "F.Cu") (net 27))
 (segment (start 179.5453 106.9032) (end 178.7374 106.0953) (width 0.25) (layer "F.Cu") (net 27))
 (segment (start 175.1435 109.0961) (end 178.4159 109.0961) (width 0.25) (layer "F.Cu") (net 27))
 (segment (start 165.6547 98.24) (end 165.6547 99.6073) (width 0.25) (layer "F.Cu") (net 27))
 (segment (start 178.37 104.92) (end 178.37 106.0953) (width 0.25) (layer "F.Cu") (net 27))
 (segment (start 178.4159 109.0961) (end 179.5453 107.9667) (width 0.25) (layer "F.Cu") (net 27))
 (segment (start 174.5853 104.92) (end 175.83 104.92) (width 0.25) (layer "F.Cu") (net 28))
 (segment (start 166.53 97.74) (end 167.4053 97.74) (width 0.25) (layer "F.Cu") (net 28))
 (segment (start 167.4053 97.74) (end 174.5853 104.92) (width 0.25) (layer "F.Cu") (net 28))
 (segment (start 178.37 102.38) (end 177.1947 102.38) (width 0.25) (layer "F.Cu") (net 29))
 (segment (start 166.53 97.24) (end 167.5422 97.24) (width 0.25) (layer "F.Cu") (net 29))
 (segment (start 173.8575 103.5553) (end 176.3868 103.5553) (width 0.25) (layer "F.Cu") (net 29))
 (segment (start 177.1947 102.7474) (end 177.1947 102.38) (width 0.25) (layer "F.Cu") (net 29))
 (segment (start 176.3868 103.5553) (end 177.1947 102.7474) (width 0.25) (layer "F.Cu") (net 29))
 (segment (start 167.5422 97.24) (end 173.8575 103.5553) (width 0.25) (layer "F.Cu") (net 29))
 (segment (start 175.83 102.38) (end 173.6822 102.38) (width 0.25) (layer "F.Cu") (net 30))
 (segment (start 168.0422 96.74) (end 167.4053 96.74) (width 0.25) (layer "F.Cu") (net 30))
 (segment (start 166.53 96.74) (end 167.4053 96.74) (width 0.25) (layer "F.Cu") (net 30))
 (segment (start 173.6822 102.38) (end 168.0422 96.74) (width 0.25) (layer "F.Cu") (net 30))
 (segment (start 176.3573 101.0447) (end 172.9838 101.0447) (width 0.25) (layer "F.Cu") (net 31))
 (segment (start 172.9838 101.0447) (end 168.1791 96.24) (width 0.25) (layer "F.Cu") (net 31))
 (segment (start 177.1947 100.2073) (end 176.3573 101.0447) (width 0.25) (layer "F.Cu") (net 31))
 (segment (start 177.1947 99.84) (end 177.1947 100.2073) (width 0.25) (layer "F.Cu") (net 31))
 (segment (start 168.1791 96.24) (end 166.53 96.24) (width 0.25) (layer "F.Cu") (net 31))
 (segment (start 178.37 99.84) (end 177.1947 99.84) (width 0.25) (layer "F.Cu") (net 31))
 (segment (start 172.416 99.84) (end 168.316 95.74) (width 0.25) (layer "F.Cu") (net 32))
 (segment (start 168.316 95.74) (end 166.53 95.74) (width 0.25) (layer "F.Cu") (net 32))
 (segment (start 175.83 99.84) (end 172.416 99.84) (width 0.25) (layer "F.Cu") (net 32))
 (segment (start 177.1947 97.3) (end 177.1947 97.6674) (width 0.25) (layer "F.Cu") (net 33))
 (segment (start 176.3868 98.4753) (end 171.6882 98.4753) (width 0.25) (layer "F.Cu") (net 33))
 (segment (start 171.6882 98.4753) (end 168.4529 95.24) (width 0.25) (layer "F.Cu") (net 33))
 (segment (start 178.37 97.3) (end 177.1947 97.3) (width 0.25) (layer "F.Cu") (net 33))
 (segment (start 168.4529 95.24) (end 167.4053 95.24) (width 0.25) (layer "F.Cu") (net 33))
 (segment (start 166.53 95.24) (end 167.4053 95.24) (width 0.25) (layer "F.Cu") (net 33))
 (segment (start 177.1947 97.6674) (end 176.3868 98.4753) (width 0.25) (layer "F.Cu") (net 33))
 (segment (start 168.5898 94.74) (end 166.53 94.74) (width 0.25) (layer "F.Cu") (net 34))
 (segment (start 171.1498 97.3) (end 168.5898 94.74) (width 0.25) (layer "F.Cu") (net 34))
 (segment (start 175.83 97.3) (end 171.1498 97.3) (width 0.25) (layer "F.Cu") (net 34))
 (segment (start 177.1947 95.1274) (end 176.3868 95.9353) (width 0.25) (layer "F.Cu") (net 35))
 (segment (start 169.4661 94.24) (end 166.53 94.24) (width 0.25) (layer "F.Cu") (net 35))
 (segment (start 178.37 94.76) (end 177.1947 94.76) (width 0.25) (layer "F.Cu") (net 35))
 (segment (start 177.1947 94.76) (end 177.1947 95.1274) (width 0.25) (layer "F.Cu") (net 35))
 (segment (start 176.3868 95.9353) (end 171.1614 95.9353) (width 0.25) (layer "F.Cu") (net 35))
 (segment (start 171.1614 95.9353) (end 169.4661 94.24) (width 0.25) (layer "F.Cu") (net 35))
 (segment (start 169.6579 93.74) (end 166.53 93.74) (width 0.25) (layer "F.Cu") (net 36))
 (segment (start 170.6779 94.76) (end 169.6579 93.74) (width 0.25) (layer "F.Cu") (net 36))
 (segment (start 175.83 94.76) (end 170.6779 94.76) (width 0.25) (layer "F.Cu") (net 36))
 (segment (start 177.1947 92.22) (end 177.1947 92.5874) (width 0.25) (layer "F.Cu") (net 37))
 (segment (start 176.3868 93.3953) (end 169.9501 93.3953) (width 0.25) (layer "F.Cu") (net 37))
 (segment (start 169.9501 93.3953) (end 169.7948 93.24) (width 0.25) (layer "F.Cu") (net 37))
 (segment (start 169.7948 93.24) (end 166.53 93.24) (width 0.25) (layer "F.Cu") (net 37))
 (segment (start 177.1947 92.5874) (end 176.3868 93.3953) (width 0.25) (layer "F.Cu") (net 37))
 (segment (start 178.37 92.22) (end 177.1947 92.22) (width 0.25) (layer "F.Cu") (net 37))
 (segment (start 175.83 92.22) (end 174.6547 92.22) (width 0.25) (layer "F.Cu") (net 38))
 (segment (start 174.1347 92.74) (end 166.53 92.74) (width 0.25) (layer "F.Cu") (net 38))
 (segment (start 174.6547 92.22) (end 174.1347 92.74) (width 0.25) (layer "F.Cu") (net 38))
 (segment (start 174.5991 90.8553) (end 173.2144 92.24) (width 0.25) (layer "F.Cu") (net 39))
 (segment (start 177.1947 89.68) (end 177.1947 90.0474) (width 0.25) (layer "F.Cu") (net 39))
 (segment (start 178.37 89.68) (end 177.1947 89.68) (width 0.25) (layer "F.Cu") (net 39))
 (segment (start 177.1947 90.0474) (end 176.3868 90.8553) (width 0.25) (layer "F.Cu") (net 39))
 (segment (start 176.3868 90.8553) (end 174.5991 90.8553) (width 0.25) (layer "F.Cu") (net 39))
 (segment (start 173.2144 92.24) (end 166.53 92.24) (width 0.25) (layer "F.Cu") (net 39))
 (segment (start 166.53 91.74) (end 167.4053 91.74) (width 0.25) (layer "F.Cu") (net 40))
 (segment (start 174.6547 89.68) (end 172.5947 91.74) (width 0.25) (layer "F.Cu") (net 40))
 (segment (start 175.83 89.68) (end 174.6547 89.68) (width 0.25) (layer "F.Cu") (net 40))
 (segment (start 172.5947 91.74) (end 167.4053 91.74) (width 0.25) (layer "F.Cu") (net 40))
 (segment (start 176.3868 88.3153) (end 174.5992 88.3153) (width 0.25) (layer "F.Cu") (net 41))
 (segment (start 174.5992 88.3153) (end 171.6745 91.24) (width 0.25) (layer "F.Cu") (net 41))
 (segment (start 177.1947 87.5074) (end 176.3868 88.3153) (width 0.25) (layer "F.Cu") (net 41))
 (segment (start 178.37 87.14) (end 177.1947 87.14) (width 0.25) (layer "F.Cu") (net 41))
 (segment (start 171.6745 91.24) (end 166.53 91.24) (width 0.25) (layer "F.Cu") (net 41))
 (segment (start 177.1947 87.14) (end 177.1947 87.5074) (width 0.25) (layer "F.Cu") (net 41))
 (segment (start 175.83 87.14) (end 174.6547 87.14) (width 0.25) (layer "F.Cu") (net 42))
 (segment (start 171.0547 90.74) (end 166.53 90.74) (width 0.25) (layer "F.Cu") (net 42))
 (segment (start 174.6547 87.14) (end 171.0547 90.74) (width 0.25) (layer "F.Cu") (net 42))
 (segment (start 176.3868 85.7753) (end 174.5992 85.7753) (width 0.25) (layer "F.Cu") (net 43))
 (segment (start 178.37 84.6) (end 177.1947 84.6) (width 0.25) (layer "F.Cu") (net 43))
 (segment (start 177.1947 84.6) (end 177.1947 84.9674) (width 0.25) (layer "F.Cu") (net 43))
 (segment (start 174.5992 85.7753) (end 170.1345 90.24) (width 0.25) (layer "F.Cu") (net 43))
 (segment (start 177.1947 84.9674) (end 176.3868 85.7753) (width 0.25) (layer "F.Cu") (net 43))
 (segment (start 170.1345 90.24) (end 166.53 90.24) (width 0.25) (layer "F.Cu") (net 43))
 (segment (start 175.83 84.6) (end 174.6547 84.6) (width 0.25) (layer "F.Cu") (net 44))
 (segment (start 174.6547 84.6) (end 169.5147 89.74) (width 0.25) (layer "F.Cu") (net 44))
 (segment (start 169.5147 89.74) (end 166.53 89.74) (width 0.25) (layer "F.Cu") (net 44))
 (segment (start 168.5944 89.24) (end 166.53 89.24) (width 0.25) (layer "F.Cu") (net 45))
 (segment (start 176.3868 83.2353) (end 174.5991 83.2353) (width 0.25) (layer "F.Cu") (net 45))
 (segment (start 177.1947 82.06) (end 177.1947 82.4274) (width 0.25) (layer "F.Cu") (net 45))
 (segment (start 177.1947 82.4274) (end 176.3868 83.2353) (width 0.25) (layer "F.Cu") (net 45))
 (segment (start 178.37 82.06) (end 177.1947 82.06) (width 0.25) (layer "F.Cu") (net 45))
 (segment (start 174.5991 83.2353) (end 168.5944 89.24) (width 0.25) (layer "F.Cu") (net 45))
 (segment (start 175.83 82.06) (end 174.6547 82.06) (width 0.25) (layer "F.Cu") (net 46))
 (segment (start 174.6547 82.06) (end 167.9747 88.74) (width 0.25) (layer "F.Cu") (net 46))
 (segment (start 167.9747 88.74) (end 166.53 88.74) (width 0.25) (layer "F.Cu") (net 46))
 (segment (start 178.37 79.52) (end 177.1947 79.52) (width 0.25) (layer "F.Cu") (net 47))
 (segment (start 176.8275 80.6953) (end 177.1947 80.3281) (width 0.25) (layer "F.Cu") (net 47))
 (segment (start 167.5422 88.24) (end 175.0869 80.6953) (width 0.25) (layer "F.Cu") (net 47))
 (segment (start 166.53 88.24) (end 167.5422 88.24) (width 0.25) (layer "F.Cu") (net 47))
 (segment (start 175.0869 80.6953) (end 176.8275 80.6953) (width 0.25) (layer "F.Cu") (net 47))
 (segment (start 177.1947 80.3281) (end 177.1947 79.52) (width 0.25) (layer "F.Cu") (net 47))
 (segment (start 166.53 87.74) (end 167.4053 87.74) (width 0.25) (layer "F.Cu") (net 48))
 (segment (start 175.83 79.52) (end 174.6547 79.52) (width 0.25) (layer "F.Cu") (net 48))
 (segment (start 167.4053 86.7694) (end 167.4053 87.74) (width 0.25) (layer "F.Cu") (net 48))
 (segment (start 174.6547 79.52) (end 167.4053 86.7694) (width 0.25) (layer "F.Cu") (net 48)))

